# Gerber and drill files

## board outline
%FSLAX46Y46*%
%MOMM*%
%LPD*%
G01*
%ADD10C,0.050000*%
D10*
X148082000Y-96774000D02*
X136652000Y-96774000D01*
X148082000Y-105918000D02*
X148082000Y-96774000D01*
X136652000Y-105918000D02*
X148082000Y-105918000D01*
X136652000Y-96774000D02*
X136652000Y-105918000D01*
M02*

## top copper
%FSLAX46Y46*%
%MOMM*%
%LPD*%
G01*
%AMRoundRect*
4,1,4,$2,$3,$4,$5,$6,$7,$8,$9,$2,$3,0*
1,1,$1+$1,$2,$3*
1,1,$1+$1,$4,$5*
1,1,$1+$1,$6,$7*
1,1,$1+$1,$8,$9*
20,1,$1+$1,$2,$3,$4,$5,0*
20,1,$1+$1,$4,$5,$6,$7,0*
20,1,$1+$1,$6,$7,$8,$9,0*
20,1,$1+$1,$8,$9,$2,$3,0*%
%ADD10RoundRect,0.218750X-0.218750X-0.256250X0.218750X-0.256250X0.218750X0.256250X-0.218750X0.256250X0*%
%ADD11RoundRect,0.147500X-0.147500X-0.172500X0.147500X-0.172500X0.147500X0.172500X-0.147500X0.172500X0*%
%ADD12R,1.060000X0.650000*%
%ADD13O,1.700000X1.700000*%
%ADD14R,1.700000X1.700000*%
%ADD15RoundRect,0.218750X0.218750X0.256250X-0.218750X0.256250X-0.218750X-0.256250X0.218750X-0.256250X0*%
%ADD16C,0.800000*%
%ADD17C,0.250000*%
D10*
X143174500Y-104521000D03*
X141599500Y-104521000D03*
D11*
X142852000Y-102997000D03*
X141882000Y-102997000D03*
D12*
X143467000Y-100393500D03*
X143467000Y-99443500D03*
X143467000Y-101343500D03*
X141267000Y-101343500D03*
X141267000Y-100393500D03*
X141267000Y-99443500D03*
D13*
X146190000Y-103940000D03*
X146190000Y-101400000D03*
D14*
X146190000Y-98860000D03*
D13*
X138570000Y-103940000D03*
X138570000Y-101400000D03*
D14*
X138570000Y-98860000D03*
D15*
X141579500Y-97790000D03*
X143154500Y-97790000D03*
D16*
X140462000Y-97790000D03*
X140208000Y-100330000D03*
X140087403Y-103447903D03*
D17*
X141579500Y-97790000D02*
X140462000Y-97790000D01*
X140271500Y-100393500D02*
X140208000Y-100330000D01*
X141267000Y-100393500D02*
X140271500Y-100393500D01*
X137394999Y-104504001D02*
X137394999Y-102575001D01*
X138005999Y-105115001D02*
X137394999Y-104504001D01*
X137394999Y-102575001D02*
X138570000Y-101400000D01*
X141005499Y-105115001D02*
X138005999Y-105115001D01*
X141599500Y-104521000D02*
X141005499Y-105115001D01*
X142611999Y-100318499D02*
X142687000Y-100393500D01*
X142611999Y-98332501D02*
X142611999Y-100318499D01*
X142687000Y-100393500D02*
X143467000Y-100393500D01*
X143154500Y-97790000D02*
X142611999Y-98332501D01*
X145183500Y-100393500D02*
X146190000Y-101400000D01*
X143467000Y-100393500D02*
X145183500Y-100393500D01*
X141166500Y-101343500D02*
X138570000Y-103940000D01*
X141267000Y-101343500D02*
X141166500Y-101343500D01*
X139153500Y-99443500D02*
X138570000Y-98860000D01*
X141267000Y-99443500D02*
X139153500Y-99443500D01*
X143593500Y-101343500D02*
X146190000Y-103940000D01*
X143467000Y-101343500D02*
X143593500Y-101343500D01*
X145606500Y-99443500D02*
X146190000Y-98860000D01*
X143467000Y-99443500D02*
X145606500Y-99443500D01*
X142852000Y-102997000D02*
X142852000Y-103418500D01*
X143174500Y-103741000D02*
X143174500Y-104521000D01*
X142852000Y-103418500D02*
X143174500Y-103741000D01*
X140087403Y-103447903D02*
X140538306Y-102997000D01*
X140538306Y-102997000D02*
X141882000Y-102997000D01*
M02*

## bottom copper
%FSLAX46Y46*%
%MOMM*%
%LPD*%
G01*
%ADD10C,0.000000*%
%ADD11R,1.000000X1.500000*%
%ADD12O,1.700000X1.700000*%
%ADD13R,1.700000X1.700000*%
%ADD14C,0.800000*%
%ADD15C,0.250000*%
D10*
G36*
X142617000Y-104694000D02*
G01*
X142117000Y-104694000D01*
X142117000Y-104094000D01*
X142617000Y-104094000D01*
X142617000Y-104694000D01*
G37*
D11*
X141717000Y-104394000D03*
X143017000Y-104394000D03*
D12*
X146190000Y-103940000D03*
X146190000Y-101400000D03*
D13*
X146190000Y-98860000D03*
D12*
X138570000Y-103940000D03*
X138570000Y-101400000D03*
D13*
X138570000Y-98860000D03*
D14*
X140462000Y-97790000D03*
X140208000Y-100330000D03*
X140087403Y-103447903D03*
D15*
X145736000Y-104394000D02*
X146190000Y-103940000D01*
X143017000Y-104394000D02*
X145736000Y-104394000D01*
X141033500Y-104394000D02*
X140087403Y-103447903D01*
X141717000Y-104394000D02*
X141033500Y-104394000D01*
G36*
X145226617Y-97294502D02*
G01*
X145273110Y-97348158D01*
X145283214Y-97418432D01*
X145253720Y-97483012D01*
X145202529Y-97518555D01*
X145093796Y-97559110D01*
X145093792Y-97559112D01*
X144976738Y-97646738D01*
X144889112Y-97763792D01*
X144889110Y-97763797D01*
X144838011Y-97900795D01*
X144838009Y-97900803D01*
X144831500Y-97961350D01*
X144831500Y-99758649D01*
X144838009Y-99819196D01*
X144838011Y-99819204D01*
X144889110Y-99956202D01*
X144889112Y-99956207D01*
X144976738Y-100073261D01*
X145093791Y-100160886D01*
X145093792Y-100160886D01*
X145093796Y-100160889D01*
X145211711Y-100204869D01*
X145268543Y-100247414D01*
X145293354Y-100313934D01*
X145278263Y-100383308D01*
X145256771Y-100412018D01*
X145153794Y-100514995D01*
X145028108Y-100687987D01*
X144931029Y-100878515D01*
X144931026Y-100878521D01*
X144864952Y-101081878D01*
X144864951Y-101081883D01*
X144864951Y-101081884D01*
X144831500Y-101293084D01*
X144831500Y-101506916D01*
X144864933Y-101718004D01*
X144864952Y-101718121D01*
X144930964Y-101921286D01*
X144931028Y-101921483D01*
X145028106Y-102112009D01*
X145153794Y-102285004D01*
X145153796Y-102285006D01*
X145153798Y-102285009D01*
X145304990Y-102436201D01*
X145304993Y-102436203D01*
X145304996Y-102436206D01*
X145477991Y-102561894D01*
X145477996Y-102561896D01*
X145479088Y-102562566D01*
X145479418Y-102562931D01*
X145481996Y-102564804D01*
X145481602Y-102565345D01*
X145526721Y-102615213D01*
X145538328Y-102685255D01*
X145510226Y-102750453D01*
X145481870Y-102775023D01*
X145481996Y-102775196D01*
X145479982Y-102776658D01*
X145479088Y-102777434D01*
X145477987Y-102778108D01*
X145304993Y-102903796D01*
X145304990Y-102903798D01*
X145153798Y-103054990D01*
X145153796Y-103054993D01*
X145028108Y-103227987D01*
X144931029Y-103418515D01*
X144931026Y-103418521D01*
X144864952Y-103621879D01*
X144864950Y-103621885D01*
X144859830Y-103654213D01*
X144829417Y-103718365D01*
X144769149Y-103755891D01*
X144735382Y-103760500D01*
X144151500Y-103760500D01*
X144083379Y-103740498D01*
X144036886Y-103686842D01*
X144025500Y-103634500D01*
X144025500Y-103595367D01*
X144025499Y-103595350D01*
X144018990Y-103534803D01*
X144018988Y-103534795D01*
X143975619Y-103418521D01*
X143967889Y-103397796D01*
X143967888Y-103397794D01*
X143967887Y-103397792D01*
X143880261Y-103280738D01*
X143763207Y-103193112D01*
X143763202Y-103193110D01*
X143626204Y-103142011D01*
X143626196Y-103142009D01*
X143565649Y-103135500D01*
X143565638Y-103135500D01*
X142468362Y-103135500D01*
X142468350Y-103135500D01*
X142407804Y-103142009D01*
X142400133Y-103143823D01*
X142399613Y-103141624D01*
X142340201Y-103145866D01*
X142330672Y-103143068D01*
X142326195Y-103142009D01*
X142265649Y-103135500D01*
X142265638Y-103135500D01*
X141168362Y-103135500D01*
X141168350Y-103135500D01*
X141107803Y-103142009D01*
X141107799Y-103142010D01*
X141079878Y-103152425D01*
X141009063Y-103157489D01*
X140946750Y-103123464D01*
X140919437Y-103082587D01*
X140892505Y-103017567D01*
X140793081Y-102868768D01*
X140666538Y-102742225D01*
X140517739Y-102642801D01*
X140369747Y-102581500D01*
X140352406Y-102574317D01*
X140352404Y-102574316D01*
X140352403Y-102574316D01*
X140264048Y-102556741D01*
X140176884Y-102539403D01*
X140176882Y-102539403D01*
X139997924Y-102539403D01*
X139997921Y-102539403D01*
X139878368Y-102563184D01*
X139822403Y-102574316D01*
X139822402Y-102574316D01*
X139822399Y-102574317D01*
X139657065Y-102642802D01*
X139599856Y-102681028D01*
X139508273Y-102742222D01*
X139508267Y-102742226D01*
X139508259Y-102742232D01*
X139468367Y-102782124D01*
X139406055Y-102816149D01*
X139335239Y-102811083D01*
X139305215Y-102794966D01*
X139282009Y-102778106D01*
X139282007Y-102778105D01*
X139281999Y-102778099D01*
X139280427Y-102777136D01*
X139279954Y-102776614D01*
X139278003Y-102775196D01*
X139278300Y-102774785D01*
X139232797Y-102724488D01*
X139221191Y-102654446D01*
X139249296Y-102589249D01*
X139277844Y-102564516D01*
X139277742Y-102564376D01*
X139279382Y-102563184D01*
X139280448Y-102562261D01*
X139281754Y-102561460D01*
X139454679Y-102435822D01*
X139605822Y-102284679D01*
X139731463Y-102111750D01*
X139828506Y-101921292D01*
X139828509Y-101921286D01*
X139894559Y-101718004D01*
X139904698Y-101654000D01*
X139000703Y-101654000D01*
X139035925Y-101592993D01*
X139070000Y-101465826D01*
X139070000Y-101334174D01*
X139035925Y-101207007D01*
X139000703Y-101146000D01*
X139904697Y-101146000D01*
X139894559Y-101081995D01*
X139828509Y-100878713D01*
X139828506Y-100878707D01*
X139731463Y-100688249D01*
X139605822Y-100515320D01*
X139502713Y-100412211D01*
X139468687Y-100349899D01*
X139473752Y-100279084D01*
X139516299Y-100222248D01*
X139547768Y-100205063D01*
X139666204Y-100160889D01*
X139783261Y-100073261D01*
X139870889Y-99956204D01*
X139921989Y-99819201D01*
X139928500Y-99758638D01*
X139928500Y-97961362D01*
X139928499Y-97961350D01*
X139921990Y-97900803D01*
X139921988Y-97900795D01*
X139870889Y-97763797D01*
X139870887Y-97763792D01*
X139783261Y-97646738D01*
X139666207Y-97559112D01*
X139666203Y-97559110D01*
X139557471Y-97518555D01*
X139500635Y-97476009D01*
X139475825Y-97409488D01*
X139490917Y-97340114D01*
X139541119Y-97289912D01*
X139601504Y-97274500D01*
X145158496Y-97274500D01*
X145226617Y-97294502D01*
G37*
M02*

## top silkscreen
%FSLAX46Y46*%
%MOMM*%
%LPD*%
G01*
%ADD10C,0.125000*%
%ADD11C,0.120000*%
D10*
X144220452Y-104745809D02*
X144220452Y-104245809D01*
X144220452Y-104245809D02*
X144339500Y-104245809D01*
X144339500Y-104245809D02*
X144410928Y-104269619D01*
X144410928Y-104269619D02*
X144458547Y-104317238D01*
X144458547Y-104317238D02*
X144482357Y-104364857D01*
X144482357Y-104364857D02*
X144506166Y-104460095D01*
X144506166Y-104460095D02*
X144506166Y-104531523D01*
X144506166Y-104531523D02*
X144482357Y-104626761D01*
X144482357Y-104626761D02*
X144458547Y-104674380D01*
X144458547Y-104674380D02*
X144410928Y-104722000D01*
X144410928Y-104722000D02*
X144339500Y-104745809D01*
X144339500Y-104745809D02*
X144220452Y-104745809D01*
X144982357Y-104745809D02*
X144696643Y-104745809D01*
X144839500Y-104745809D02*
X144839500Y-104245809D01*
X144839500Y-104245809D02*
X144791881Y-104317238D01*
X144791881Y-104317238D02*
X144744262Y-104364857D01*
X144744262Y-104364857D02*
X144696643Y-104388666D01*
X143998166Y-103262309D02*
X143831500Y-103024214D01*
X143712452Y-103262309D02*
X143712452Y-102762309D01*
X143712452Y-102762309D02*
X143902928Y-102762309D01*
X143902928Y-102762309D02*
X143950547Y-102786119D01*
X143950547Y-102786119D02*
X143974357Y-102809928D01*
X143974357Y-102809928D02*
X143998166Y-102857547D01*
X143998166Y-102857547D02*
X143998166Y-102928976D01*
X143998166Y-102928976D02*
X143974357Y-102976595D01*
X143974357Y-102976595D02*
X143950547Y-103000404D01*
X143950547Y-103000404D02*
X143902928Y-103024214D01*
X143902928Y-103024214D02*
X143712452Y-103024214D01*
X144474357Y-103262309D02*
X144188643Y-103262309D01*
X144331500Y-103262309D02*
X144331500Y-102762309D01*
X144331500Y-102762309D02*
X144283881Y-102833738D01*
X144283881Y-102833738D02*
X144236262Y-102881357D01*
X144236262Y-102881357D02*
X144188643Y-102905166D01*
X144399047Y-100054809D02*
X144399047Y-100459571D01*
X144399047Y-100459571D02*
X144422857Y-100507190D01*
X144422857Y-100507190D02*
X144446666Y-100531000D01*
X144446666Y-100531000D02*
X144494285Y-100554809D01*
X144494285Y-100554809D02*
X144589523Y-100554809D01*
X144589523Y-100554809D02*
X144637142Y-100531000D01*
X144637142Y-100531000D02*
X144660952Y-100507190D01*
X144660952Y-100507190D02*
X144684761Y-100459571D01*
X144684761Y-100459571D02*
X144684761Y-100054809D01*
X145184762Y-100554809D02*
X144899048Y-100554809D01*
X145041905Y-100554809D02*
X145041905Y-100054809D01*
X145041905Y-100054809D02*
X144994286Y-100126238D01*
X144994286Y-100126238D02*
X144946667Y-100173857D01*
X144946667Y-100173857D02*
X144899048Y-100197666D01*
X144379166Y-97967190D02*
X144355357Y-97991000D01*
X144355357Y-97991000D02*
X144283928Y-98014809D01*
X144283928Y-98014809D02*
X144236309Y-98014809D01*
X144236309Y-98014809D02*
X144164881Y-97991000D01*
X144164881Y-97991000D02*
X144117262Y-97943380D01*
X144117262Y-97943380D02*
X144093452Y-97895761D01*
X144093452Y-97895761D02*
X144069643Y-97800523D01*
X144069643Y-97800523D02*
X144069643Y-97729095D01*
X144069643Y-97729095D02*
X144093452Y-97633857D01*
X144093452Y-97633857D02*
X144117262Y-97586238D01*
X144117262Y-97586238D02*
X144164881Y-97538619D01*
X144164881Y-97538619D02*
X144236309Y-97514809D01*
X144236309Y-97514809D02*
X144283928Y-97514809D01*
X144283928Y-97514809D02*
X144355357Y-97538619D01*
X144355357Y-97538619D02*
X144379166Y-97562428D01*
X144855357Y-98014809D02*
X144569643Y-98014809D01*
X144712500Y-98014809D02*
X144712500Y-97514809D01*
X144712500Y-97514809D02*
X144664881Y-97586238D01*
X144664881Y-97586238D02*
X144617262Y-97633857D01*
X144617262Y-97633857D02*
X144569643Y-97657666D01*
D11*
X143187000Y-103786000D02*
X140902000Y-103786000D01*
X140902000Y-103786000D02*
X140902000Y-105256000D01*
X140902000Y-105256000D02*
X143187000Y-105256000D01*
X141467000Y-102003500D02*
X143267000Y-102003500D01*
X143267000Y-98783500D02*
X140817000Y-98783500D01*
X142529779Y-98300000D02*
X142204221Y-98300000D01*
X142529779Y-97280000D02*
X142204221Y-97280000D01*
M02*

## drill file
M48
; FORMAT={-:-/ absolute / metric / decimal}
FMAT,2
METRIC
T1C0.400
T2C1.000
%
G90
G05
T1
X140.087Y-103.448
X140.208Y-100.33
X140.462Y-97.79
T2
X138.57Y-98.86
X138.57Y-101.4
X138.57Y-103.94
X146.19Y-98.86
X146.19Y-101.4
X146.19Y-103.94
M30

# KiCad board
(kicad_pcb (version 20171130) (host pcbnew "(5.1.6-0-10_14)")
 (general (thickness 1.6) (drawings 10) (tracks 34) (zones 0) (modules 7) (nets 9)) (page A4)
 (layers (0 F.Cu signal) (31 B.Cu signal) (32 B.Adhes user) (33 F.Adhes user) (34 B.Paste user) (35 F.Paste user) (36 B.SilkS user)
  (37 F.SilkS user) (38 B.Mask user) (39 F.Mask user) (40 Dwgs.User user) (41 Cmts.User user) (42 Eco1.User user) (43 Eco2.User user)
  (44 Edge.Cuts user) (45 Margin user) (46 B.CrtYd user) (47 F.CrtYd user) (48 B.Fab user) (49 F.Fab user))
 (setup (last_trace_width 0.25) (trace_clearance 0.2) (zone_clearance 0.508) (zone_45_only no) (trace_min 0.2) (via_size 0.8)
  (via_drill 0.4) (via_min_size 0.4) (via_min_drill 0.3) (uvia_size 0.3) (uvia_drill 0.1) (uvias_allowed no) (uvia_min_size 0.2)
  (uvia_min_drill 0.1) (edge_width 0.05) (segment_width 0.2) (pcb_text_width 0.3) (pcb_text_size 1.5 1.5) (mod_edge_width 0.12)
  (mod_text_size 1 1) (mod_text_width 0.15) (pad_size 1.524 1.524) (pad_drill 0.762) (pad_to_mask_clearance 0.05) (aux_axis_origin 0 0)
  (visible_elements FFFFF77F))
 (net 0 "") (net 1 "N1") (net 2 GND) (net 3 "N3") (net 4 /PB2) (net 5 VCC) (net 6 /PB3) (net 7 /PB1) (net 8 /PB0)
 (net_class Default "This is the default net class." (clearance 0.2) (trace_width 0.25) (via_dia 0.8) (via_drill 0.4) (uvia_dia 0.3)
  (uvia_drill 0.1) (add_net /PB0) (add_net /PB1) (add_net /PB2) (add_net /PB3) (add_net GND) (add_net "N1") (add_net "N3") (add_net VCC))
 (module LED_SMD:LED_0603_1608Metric (layer F.Cu) (at 142.387 104.521)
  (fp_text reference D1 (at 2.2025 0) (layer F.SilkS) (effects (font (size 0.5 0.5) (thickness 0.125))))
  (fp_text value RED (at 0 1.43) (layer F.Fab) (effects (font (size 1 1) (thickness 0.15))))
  (fp_line (start 0.8 -0.735) (end -1.485 -0.735) (layer F.SilkS) (width 0.12))
  (fp_line (start -1.485 -0.735) (end -1.485 0.735) (layer F.SilkS) (width 0.12))
  (fp_line (start -1.485 0.735) (end 0.8 0.735) (layer F.SilkS) (width 0.12))
  (pad 2 smd roundrect (at 0.7875 0) (size 0.875 0.95) (layers F.Cu F.Paste F.Mask) (roundrect_rratio 0.25) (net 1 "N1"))
  (pad 1 smd roundrect (at -0.7875 0) (size 0.875 0.95) (layers F.Cu F.Paste F.Mask) (roundrect_rratio 0.25) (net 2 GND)))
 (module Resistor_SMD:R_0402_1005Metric (layer F.Cu) (at 142.367 102.997)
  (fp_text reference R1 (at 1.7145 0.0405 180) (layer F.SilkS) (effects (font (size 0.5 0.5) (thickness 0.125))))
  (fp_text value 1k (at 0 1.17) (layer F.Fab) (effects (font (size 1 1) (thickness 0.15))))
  (pad 2 smd roundrect (at 0.485 0) (size 0.59 0.64) (layers F.Cu F.Paste F.Mask) (roundrect_rratio 0.25) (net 1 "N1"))
  (pad 1 smd roundrect (at -0.485 0) (size 0.59 0.64) (layers F.Cu F.Paste F.Mask) (roundrect_rratio 0.25) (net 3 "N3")))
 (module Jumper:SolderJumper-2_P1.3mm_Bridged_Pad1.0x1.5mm (layer B.Cu) (at 142.367 104.394 180)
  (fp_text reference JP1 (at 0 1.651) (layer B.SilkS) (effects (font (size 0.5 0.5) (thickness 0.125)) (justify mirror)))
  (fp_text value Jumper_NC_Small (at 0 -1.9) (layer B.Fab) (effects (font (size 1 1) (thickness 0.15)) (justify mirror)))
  (fp_poly (pts (xy -0.25 0.3) (xy 0.25 0.3) (xy 0.25 -0.3) (xy -0.25 -0.3)) (layer B.Cu) (width 0))
  (pad 2 smd rect (at 0.65 0 180) (size 1 1.5) (layers B.Cu B.Mask) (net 3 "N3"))
  (pad 1 smd rect (at -0.65 0 180) (size 1 1.5) (layers B.Cu B.Mask) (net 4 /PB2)))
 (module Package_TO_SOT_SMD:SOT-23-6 (layer F.Cu) (at 142.367 100.3935)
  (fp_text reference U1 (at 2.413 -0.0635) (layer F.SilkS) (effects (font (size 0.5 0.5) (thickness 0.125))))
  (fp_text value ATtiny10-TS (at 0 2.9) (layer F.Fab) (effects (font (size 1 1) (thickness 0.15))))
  (fp_line (start -0.9 1.61) (end 0.9 1.61) (layer F.SilkS) (width 0.12))
  (fp_line (start 0.9 -1.61) (end -1.55 -1.61) (layer F.SilkS) (width 0.12))
  (pad 5 smd rect (at 1.1 0) (size 1.06 0.65) (layers F.Cu F.Paste F.Mask) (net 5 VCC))
  (pad 6 smd rect (at 1.1 -0.95) (size 1.06 0.65) (layers F.Cu F.Paste F.Mask) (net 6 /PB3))
  (pad 4 smd rect (at 1.1 0.95) (size 1.06 0.65) (layers F.Cu F.Paste F.Mask) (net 4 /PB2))
  (pad 3 smd rect (at -1.1 0.95) (size 1.06 0.65) (layers F.Cu F.Paste F.Mask) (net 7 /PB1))
  (pad 2 smd rect (at -1.1 0) (size 1.06 0.65) (layers F.Cu F.Paste F.Mask) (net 2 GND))
  (pad 1 smd rect (at -1.1 -0.95) (size 1.06 0.65) (layers F.Cu F.Paste F.Mask) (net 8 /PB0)))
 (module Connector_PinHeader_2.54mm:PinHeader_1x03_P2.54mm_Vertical (layer B.Cu) (at 146.19 98.86 180)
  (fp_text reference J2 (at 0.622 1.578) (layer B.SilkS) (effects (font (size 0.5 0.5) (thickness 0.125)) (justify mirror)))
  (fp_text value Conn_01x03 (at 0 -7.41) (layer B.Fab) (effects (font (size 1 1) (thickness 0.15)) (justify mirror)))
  (pad 3 thru_hole oval (at 0 -5.08 180) (size 1.7 1.7) (drill 1) (layers *.Cu *.Mask) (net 4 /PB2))
  (pad 2 thru_hole oval (at 0 -2.54 180) (size 1.7 1.7) (drill 1) (layers *.Cu *.Mask) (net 5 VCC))
  (pad 1 thru_hole rect (at 0 0 180) (size 1.7 1.7) (drill 1) (layers *.Cu *.Mask) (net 6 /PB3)))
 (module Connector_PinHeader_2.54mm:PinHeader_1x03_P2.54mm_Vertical (layer B.Cu) (at 138.57 98.86 180)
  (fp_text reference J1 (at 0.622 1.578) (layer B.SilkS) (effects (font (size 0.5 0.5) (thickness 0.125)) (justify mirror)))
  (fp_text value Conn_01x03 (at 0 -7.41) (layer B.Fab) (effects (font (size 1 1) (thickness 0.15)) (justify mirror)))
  (pad 3 thru_hole oval (at 0 -5.08 180) (size 1.7 1.7) (drill 1) (layers *.Cu *.Mask) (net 7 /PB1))
  (pad 2 thru_hole oval (at 0 -2.54 180) (size 1.7 1.7) (drill 1) (layers *.Cu *.Mask) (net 2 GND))
  (pad 1 thru_hole rect (at 0 0 180) (size 1.7 1.7) (drill 1) (layers *.Cu *.Mask) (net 8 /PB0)))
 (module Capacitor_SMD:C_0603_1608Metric (layer F.Cu) (at 142.367 97.79 180)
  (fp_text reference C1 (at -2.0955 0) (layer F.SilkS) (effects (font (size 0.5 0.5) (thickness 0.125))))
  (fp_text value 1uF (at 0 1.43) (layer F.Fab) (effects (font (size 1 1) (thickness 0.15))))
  (fp_line (start -0.162779 -0.51) (end 0.162779 -0.51) (layer F.SilkS) (width 0.12))
  (fp_line (start -0.162779 0.51) (end 0.162779 0.51) (layer F.SilkS) (width 0.12))
  (pad 2 smd roundrect (at 0.7875 0 180) (size 0.875 0.95) (layers F.Cu F.Paste F.Mask) (roundrect_rratio 0.25) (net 2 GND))
  (pad 1 smd roundrect (at -0.7875 0 180) (size 0.875 0.95) (layers F.Cu F.Paste F.Mask) (roundrect_rratio 0.25) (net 5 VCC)))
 (gr_line (start 148.082 96.774) (end 136.652 96.774) (layer Edge.Cuts) (width 0.05))
 (gr_line (start 148.082 105.918) (end 148.082 96.774) (layer Edge.Cuts) (width 0.05))
 (gr_line (start 136.652 105.918) (end 148.082 105.918) (layer Edge.Cuts) (width 0.05))
 (gr_line (start 136.652 96.774) (end 136.652 105.918) (layer Edge.Cuts) (width 0.05))
 (via (at 140.462 97.79) (size 0.8) (drill 0.4) (layers F.Cu B.Cu) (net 2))
 (segment (start 141.5795 97.79) (end 140.462 97.79) (width 0.25) (layer F.Cu) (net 2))
 (via (at 140.208 100.33) (size 0.8) (drill 0.4) (layers F.Cu B.Cu) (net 2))
 (segment (start 140.2715 100.3935) (end 140.208 100.33) (width 0.25) (layer F.Cu) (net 2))
 (segment (start 141.267 100.3935) (end 140.2715 100.3935) (width 0.25) (layer F.Cu) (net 2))
 (segment (start 137.394999 104.504001) (end 137.394999 102.575001) (width 0.25) (layer F.Cu) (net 2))
 (segment (start 138.005999 105.115001) (end 137.394999 104.504001) (width 0.25) (layer F.Cu) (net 2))
 (segment (start 137.394999 102.575001) (end 138.57 101.4) (width 0.25) (layer F.Cu) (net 2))
 (segment (start 141.005499 105.115001) (end 138.005999 105.115001) (width 0.25) (layer F.Cu) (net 2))
 (segment (start 141.5995 104.521) (end 141.005499 105.115001) (width 0.25) (layer F.Cu) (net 2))
 (segment (start 142.611999 100.318499) (end 142.687 100.3935) (width 0.25) (layer F.Cu) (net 5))
 (segment (start 142.611999 98.332501) (end 142.611999 100.318499) (width 0.25) (layer F.Cu) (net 5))
 (segment (start 142.687 100.3935) (end 143.467 100.3935) (width 0.25) (layer F.Cu) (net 5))
 (segment (start 143.1545 97.79) (end 142.611999 98.332501) (width 0.25) (layer F.Cu) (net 5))
 (segment (start 145.1835 100.3935) (end 146.19 101.4) (width 0.25) (layer F.Cu) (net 5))
 (segment (start 143.467 100.3935) (end 145.1835 100.3935) (width 0.25) (layer F.Cu) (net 5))
 (segment (start 141.1665 101.3435) (end 138.57 103.94) (width 0.25) (layer F.Cu) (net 7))
 (segment (start 141.267 101.3435) (end 141.1665 101.3435) (width 0.25) (layer F.Cu) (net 7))
 (segment (start 139.1535 99.4435) (end 138.57 98.86) (width 0.25) (layer F.Cu) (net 8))
 (segment (start 141.267 99.4435) (end 139.1535 99.4435) (width 0.25) (layer F.Cu) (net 8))
 (segment (start 143.5935 101.3435) (end 146.19 103.94) (width 0.25) (layer F.Cu) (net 4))
 (segment (start 143.467 101.3435) (end 143.5935 101.3435) (width 0.25) (layer F.Cu) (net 4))
 (segment (start 145.736 104.394) (end 146.19 103.94) (width 0.25) (layer B.Cu) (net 4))
 (segment (start 143.017 104.394) (end 145.736 104.394) (width 0.25) (layer B.Cu) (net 4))
 (segment (start 145.6065 99.4435) (end 146.19 98.86) (width 0.25) (layer F.Cu) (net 6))
 (segment (start 143.467 99.4435) (end 145.6065 99.4435) (width 0.25) (layer F.Cu) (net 6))
 (segment (start 142.852 102.997) (end 142.852 103.4185) (width 0.25) (layer F.Cu) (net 1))
 (segment (start 143.1745 103.741) (end 143.1745 104.521) (width 0.25) (layer F.Cu) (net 1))
 (segment (start 142.852 103.4185) (end 143.1745 103.741) (width 0.25) (layer F.Cu) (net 1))
 (via (at 140.087403 103.447903) (size 0.8) (drill 0.4) (layers F.Cu B.Cu) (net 3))
 (segment (start 141.0335 104.394) (end 140.087403 103.447903) (width 0.25) (layer B.Cu) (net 3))
 (segment (start 141.717 104.394) (end 141.0335 104.394) (width 0.25) (layer B.Cu) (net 3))
 (segment (start 140.087403 103.447903) (end 140.538306 102.997) (width 0.25) (layer F.Cu) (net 3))
 (segment (start 140.538306 102.997) (end 141.882 102.997) (width 0.25) (layer F.Cu) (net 3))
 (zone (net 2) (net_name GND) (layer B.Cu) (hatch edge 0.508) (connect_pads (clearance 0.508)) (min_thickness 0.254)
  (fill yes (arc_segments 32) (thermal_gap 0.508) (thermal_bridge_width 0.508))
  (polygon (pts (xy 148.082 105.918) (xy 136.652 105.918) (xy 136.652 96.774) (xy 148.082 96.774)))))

